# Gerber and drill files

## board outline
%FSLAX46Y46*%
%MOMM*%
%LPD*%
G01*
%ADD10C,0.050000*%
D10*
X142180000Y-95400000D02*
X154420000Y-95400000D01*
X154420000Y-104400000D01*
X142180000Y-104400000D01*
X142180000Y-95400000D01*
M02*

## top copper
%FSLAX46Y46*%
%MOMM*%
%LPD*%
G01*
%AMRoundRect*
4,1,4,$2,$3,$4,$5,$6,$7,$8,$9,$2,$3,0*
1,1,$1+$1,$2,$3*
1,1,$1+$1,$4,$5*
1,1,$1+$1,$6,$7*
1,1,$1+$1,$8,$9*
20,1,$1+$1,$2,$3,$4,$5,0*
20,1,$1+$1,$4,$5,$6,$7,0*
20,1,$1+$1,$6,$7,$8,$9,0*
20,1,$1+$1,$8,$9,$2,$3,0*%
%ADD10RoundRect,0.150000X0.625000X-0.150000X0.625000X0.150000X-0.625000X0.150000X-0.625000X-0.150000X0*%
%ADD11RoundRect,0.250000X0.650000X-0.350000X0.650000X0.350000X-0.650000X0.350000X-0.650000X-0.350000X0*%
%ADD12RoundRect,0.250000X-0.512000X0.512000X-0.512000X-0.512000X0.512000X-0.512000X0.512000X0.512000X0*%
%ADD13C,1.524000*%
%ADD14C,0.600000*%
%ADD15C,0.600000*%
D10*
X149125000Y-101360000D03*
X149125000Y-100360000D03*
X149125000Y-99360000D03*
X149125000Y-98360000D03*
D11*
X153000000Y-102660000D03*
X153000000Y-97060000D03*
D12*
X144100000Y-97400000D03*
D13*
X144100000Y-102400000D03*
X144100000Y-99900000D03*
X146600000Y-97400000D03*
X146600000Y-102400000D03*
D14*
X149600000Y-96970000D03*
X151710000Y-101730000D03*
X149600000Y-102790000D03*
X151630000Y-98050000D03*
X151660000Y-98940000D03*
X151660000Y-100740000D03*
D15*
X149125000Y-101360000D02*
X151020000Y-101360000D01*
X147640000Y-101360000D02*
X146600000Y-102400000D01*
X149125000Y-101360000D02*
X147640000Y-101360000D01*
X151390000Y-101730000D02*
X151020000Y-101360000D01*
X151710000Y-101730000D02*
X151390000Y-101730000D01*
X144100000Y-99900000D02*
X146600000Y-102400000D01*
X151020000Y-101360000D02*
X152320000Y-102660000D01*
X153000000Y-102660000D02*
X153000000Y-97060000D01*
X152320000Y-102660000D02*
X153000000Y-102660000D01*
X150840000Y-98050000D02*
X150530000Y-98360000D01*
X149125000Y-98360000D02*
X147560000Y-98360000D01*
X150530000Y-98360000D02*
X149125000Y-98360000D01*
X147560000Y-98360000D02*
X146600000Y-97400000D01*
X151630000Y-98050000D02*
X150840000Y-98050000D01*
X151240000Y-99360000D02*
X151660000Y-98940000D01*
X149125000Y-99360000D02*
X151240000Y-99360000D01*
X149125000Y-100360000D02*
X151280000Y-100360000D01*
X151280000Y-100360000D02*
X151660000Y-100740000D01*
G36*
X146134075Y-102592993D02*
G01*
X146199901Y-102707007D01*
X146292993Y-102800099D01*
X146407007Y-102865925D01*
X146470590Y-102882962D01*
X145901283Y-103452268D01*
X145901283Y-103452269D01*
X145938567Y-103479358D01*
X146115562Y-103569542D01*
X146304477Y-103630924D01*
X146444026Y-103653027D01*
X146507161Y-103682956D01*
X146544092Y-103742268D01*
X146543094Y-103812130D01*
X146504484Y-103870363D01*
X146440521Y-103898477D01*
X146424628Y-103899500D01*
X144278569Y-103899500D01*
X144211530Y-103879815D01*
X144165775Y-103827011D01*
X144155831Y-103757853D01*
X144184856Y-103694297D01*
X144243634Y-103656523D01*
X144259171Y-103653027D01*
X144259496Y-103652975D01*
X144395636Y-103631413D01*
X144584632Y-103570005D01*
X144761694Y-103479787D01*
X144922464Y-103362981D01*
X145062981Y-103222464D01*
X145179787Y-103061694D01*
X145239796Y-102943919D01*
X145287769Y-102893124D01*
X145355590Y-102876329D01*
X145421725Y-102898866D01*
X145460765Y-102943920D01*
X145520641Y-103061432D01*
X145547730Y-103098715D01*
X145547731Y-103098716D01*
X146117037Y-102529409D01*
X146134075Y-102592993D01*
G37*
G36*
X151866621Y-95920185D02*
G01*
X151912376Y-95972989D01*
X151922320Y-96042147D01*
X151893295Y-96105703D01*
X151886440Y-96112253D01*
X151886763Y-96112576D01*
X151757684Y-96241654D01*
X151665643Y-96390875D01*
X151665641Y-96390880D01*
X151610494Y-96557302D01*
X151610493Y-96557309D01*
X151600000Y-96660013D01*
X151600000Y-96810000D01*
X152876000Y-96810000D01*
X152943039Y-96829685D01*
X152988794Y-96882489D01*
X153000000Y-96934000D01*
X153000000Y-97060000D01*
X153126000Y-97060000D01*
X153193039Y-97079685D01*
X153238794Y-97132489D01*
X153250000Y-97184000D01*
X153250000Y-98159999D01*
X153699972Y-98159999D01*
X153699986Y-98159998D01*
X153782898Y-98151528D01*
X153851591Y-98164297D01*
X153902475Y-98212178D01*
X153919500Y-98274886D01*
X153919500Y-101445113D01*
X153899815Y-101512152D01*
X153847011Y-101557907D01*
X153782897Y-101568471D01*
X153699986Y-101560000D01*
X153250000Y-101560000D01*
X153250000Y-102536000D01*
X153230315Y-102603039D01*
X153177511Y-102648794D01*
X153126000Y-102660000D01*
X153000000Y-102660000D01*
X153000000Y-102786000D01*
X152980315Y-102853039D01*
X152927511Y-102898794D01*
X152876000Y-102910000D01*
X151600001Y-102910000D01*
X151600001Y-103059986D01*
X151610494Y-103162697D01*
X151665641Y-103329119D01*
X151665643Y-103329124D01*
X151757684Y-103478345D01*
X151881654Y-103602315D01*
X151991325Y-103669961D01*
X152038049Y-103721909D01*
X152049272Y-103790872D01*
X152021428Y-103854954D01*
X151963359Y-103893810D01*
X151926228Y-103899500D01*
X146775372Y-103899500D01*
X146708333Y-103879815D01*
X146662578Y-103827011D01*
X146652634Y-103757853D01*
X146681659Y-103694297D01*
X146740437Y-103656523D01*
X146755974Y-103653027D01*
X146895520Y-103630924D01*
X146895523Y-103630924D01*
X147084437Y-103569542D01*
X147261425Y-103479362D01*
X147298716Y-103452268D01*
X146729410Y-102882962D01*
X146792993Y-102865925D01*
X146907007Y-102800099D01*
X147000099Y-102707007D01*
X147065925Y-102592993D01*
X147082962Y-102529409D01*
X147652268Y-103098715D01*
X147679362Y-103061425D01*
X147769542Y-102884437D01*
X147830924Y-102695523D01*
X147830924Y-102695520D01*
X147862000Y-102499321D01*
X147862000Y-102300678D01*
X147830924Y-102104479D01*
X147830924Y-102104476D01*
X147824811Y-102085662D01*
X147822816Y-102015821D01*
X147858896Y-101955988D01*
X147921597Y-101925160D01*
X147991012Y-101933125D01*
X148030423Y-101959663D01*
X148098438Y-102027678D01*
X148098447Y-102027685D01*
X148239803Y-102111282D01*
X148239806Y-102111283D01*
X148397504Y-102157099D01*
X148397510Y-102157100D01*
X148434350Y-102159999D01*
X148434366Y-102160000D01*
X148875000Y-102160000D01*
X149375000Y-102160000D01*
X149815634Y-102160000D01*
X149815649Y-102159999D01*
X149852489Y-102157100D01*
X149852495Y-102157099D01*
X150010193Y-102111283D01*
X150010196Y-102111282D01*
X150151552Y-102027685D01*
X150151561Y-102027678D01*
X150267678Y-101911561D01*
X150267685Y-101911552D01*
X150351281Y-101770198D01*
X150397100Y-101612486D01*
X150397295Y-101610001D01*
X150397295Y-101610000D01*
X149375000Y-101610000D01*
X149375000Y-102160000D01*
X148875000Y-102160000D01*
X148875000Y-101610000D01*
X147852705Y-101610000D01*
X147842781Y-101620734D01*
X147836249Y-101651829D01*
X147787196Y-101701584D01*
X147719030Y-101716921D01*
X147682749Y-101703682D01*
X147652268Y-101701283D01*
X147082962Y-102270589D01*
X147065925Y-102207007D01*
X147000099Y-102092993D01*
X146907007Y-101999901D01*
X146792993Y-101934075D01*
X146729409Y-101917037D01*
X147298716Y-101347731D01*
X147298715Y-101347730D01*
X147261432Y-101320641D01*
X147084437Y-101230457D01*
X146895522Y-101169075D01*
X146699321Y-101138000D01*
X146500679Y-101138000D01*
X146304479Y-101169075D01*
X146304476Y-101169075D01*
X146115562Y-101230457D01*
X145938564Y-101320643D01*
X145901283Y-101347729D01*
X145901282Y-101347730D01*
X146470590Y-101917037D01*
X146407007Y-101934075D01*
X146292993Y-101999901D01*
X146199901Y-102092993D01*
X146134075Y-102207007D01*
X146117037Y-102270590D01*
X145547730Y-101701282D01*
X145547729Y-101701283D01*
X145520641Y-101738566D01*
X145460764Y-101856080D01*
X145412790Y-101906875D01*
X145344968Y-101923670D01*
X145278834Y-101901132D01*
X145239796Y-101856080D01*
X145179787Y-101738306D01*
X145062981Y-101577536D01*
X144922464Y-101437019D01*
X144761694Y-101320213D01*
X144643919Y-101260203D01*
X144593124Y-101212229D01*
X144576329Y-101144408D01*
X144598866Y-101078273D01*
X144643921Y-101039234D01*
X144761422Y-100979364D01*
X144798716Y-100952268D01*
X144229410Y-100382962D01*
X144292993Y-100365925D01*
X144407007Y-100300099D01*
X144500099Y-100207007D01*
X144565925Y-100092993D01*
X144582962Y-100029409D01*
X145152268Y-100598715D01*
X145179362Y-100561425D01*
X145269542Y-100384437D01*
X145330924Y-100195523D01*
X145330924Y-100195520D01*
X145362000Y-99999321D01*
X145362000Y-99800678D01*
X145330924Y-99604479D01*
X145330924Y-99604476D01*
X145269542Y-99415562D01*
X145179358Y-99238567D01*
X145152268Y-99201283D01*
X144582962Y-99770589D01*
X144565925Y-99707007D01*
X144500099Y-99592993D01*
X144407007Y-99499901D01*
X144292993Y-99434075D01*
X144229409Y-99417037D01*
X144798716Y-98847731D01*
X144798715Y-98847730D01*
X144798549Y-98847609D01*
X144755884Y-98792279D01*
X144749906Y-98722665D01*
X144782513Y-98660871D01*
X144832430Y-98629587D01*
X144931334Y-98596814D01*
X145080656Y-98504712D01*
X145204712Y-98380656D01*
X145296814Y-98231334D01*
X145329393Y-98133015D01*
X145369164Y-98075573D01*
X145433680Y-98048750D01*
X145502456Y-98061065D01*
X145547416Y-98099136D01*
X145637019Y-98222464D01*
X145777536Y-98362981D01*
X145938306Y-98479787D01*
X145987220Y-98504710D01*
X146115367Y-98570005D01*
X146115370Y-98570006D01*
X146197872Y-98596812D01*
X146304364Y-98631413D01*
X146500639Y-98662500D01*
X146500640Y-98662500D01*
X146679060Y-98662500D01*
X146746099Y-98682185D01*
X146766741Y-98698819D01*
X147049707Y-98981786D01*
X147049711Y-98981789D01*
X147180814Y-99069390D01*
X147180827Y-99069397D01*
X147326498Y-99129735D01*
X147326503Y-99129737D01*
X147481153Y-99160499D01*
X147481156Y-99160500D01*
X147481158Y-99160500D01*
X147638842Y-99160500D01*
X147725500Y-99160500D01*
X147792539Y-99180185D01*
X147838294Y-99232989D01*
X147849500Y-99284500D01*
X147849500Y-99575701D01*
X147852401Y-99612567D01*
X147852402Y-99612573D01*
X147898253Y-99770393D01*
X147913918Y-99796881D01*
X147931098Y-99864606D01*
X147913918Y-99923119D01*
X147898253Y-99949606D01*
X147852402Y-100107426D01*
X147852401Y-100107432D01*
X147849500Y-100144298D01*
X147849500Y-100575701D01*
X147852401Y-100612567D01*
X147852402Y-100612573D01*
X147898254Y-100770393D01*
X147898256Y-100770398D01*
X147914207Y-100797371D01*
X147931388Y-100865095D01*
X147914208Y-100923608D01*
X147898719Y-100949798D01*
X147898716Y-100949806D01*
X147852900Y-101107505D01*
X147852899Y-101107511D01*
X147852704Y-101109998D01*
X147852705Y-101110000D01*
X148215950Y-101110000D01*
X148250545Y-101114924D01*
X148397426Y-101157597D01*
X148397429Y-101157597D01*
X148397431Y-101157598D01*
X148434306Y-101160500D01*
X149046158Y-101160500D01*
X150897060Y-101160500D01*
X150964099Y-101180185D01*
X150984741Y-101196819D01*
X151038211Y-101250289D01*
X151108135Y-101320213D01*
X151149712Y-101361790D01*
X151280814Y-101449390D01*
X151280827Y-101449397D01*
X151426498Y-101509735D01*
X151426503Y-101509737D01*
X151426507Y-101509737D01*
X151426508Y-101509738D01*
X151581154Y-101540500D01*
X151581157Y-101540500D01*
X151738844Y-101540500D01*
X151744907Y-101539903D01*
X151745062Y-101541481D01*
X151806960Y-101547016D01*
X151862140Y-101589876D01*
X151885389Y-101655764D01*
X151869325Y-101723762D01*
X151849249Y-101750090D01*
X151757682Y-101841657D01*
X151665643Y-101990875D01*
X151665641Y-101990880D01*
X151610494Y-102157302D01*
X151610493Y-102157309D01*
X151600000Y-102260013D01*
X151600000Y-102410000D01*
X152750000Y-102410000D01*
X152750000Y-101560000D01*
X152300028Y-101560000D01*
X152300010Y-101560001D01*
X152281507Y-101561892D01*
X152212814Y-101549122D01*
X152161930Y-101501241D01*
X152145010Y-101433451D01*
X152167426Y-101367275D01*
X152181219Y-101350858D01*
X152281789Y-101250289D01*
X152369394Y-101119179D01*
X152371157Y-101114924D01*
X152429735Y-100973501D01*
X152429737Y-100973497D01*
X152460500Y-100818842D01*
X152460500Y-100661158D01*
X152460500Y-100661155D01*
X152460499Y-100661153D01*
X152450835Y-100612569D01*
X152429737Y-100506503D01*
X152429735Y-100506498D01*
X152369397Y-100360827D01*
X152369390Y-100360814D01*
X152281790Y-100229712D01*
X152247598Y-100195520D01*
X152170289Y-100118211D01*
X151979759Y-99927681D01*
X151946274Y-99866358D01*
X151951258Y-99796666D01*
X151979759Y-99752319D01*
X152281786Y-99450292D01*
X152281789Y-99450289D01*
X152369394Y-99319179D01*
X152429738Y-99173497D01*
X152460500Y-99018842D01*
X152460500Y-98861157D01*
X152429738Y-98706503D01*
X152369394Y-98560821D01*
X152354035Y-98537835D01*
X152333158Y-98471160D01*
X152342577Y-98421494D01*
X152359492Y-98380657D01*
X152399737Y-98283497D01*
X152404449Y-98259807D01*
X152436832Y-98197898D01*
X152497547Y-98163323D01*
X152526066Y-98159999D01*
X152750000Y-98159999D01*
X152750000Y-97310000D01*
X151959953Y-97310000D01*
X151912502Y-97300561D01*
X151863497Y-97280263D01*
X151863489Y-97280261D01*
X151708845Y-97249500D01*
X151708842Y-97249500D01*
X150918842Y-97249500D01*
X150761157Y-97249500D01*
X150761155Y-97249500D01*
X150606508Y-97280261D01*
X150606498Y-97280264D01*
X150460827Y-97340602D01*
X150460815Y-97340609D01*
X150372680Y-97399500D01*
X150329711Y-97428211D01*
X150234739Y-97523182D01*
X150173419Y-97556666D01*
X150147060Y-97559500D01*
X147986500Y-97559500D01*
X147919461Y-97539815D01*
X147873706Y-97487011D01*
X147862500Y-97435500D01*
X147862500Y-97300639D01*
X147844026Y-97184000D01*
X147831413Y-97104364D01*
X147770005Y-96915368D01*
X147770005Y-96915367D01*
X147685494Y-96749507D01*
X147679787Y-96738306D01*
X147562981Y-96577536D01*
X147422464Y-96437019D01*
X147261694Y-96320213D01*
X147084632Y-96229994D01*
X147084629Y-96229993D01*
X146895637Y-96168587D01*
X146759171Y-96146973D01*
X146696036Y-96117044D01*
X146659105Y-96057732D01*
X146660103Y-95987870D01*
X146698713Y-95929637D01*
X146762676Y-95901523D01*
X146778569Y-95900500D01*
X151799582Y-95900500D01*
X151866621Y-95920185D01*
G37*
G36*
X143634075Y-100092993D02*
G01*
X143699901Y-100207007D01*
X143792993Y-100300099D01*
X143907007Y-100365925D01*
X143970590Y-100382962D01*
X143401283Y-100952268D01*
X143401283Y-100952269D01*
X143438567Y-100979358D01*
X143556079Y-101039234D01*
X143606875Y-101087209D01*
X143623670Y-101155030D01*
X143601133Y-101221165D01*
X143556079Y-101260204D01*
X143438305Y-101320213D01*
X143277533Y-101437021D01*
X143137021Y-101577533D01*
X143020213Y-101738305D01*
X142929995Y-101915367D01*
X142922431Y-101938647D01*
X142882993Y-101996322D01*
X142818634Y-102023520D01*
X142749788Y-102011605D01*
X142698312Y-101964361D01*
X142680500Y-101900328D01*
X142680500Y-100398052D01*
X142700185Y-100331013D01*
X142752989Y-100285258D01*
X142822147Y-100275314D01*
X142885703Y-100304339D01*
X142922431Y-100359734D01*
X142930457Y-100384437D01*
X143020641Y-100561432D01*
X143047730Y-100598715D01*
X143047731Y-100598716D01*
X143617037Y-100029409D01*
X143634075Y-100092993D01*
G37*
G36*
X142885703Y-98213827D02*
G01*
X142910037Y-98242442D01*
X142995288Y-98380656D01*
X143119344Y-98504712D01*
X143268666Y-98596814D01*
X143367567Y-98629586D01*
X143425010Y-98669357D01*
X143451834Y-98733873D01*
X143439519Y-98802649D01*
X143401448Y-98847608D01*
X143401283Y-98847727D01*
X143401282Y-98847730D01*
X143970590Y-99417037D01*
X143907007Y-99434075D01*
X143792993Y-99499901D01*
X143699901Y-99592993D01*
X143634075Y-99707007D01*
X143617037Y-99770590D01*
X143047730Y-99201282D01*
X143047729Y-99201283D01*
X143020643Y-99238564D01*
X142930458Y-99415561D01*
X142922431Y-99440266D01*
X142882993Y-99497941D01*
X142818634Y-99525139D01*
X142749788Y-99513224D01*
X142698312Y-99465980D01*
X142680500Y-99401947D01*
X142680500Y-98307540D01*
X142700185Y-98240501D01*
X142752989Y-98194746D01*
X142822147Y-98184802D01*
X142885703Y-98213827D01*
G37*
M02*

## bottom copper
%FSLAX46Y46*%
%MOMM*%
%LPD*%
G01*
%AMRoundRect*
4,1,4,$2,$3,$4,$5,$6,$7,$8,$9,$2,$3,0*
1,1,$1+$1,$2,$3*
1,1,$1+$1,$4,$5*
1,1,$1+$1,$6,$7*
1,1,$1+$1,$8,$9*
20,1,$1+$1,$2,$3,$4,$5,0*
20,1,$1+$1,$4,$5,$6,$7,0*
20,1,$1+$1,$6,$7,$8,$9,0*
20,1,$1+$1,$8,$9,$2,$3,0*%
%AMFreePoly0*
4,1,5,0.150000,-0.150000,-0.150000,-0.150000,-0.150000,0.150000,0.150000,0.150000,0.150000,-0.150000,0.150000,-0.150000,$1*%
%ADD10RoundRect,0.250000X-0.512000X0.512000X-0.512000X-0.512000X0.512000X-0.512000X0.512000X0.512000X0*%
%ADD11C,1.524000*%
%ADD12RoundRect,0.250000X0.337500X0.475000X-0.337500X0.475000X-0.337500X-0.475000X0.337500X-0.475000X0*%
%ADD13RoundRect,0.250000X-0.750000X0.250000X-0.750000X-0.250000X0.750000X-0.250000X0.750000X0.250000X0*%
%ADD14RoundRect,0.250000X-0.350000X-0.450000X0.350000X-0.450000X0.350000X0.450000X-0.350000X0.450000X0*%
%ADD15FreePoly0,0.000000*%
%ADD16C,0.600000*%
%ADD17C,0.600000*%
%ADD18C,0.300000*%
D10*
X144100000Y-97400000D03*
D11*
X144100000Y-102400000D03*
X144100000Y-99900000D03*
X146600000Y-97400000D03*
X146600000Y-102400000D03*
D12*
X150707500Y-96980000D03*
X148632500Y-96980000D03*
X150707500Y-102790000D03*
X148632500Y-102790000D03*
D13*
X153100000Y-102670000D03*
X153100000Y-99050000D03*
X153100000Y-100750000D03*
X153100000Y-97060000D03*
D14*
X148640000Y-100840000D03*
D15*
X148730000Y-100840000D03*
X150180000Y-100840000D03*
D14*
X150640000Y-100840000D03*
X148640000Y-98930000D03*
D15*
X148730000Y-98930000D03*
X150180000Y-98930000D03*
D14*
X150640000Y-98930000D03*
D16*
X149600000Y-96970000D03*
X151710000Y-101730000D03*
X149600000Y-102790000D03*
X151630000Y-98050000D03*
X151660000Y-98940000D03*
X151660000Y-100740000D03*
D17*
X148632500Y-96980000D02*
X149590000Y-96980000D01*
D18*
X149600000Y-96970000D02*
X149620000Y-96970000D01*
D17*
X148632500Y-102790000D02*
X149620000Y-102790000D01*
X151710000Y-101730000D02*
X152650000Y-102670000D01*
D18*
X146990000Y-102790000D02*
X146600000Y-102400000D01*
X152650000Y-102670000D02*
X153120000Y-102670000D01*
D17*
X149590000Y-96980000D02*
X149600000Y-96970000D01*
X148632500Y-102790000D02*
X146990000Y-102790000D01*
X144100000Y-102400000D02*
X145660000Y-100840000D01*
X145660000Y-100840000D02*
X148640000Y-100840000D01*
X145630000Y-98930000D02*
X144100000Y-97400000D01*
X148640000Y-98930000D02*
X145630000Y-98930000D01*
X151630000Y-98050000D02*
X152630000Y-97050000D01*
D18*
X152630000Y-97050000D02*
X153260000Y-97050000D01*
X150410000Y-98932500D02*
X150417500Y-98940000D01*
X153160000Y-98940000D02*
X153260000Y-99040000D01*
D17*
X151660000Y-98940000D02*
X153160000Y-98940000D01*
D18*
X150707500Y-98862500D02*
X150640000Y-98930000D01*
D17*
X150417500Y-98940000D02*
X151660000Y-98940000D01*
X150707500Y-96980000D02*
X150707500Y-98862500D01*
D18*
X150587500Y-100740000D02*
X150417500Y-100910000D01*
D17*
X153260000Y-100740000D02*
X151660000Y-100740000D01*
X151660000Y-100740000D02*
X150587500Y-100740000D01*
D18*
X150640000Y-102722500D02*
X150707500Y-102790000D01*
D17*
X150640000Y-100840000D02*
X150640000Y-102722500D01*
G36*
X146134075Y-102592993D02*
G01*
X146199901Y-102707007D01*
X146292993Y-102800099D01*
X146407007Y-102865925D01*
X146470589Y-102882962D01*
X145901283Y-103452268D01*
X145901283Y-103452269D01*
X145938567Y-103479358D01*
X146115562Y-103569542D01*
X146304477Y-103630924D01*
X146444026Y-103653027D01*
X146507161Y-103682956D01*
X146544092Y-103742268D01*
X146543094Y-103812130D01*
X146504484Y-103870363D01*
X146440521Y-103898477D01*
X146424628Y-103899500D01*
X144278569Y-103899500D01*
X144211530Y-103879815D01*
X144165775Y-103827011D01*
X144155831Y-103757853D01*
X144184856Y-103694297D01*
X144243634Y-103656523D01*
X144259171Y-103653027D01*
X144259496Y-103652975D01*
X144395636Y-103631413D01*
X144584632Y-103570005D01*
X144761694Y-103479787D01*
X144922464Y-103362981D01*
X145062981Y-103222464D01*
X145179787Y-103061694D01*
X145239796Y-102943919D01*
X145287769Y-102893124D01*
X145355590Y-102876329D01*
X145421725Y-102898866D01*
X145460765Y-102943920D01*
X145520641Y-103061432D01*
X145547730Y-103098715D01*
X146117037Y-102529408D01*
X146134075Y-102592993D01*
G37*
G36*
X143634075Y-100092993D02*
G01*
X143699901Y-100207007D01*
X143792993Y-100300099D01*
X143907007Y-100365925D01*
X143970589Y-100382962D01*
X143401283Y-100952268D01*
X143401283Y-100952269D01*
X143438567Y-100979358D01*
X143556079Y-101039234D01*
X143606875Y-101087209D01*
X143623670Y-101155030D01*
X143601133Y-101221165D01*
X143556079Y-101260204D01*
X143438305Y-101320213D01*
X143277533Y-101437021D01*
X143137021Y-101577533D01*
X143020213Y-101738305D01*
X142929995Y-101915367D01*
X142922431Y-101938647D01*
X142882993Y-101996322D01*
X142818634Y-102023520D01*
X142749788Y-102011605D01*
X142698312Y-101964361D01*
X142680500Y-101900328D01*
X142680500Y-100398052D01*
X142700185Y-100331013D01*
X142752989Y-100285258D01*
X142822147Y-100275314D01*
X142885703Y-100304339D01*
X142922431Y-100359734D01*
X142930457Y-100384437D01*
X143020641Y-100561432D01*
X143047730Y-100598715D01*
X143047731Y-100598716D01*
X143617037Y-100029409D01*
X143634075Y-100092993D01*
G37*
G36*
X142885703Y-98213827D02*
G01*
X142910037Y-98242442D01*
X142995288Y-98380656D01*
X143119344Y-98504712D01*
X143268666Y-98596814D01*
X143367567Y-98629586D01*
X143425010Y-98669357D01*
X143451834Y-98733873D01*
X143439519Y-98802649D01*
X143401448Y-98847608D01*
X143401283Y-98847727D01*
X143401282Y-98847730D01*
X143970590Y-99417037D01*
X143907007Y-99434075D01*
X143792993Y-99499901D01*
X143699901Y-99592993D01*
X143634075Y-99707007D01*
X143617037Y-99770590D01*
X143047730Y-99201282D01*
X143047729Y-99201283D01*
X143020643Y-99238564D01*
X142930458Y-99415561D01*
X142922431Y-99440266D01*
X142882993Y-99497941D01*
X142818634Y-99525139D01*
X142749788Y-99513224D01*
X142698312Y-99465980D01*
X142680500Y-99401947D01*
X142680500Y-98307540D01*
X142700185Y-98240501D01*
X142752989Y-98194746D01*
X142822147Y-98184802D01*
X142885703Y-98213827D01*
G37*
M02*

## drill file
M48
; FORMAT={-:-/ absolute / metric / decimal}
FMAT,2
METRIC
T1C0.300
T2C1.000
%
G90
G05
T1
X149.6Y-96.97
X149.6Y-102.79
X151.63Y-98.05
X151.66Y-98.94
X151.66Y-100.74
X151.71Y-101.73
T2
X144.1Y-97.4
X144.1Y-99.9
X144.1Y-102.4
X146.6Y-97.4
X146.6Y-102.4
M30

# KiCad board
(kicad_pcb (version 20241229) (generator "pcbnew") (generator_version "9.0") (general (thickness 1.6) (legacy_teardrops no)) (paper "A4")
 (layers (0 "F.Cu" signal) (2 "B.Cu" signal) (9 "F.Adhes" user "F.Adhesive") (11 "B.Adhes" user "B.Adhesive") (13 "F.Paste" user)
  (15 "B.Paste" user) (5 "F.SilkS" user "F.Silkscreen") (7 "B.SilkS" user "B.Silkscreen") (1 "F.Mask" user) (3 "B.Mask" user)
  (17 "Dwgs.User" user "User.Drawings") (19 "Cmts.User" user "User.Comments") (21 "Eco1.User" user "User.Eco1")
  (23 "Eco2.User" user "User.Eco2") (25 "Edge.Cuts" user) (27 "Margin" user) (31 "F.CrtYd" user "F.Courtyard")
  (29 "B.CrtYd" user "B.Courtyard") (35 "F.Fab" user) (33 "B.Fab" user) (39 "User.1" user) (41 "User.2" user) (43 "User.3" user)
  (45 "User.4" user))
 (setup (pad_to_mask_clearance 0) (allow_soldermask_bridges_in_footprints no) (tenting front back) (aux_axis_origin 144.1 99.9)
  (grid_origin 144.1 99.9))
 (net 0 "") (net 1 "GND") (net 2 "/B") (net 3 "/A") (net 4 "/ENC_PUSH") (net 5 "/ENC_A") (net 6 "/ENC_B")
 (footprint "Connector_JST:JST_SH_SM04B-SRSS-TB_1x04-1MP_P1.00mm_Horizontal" (layer "F.Cu") (at 151.125 99.86 90)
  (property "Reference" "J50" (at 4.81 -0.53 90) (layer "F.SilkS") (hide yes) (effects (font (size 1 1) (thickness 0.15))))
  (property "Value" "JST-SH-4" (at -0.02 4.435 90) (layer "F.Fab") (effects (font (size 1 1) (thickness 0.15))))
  (pad "1" smd roundrect (at -1.5 -2 90) (size 0.6 1.55) (layers "F.Cu" "F.Mask" "F.Paste") (roundrect_rratio 0.25) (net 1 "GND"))
  (pad "2" smd roundrect (at -0.5 -2 90) (size 0.6 1.55) (layers "F.Cu" "F.Mask" "F.Paste") (roundrect_rratio 0.25) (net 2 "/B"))
  (pad "3" smd roundrect (at 0.5 -2 90) (size 0.6 1.55) (layers "F.Cu" "F.Mask" "F.Paste") (roundrect_rratio 0.25) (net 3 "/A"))
  (pad "4" smd roundrect (at 1.5 -2 90) (size 0.6 1.55) (layers "F.Cu" "F.Mask" "F.Paste") (roundrect_rratio 0.25) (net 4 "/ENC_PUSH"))
  (pad "MP" smd roundrect (at -2.8 1.875 90) (size 1.2 1.8) (layers "F.Cu" "F.Mask" "F.Paste") (roundrect_rratio 0.208333) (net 1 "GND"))
  (pad "MP" smd roundrect (at 2.8 1.875 90) (size 1.2 1.8) (layers "F.Cu" "F.Mask" "F.Paste") (roundrect_rratio 0.208333) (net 1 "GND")))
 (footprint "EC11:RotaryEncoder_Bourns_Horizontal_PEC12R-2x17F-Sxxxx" (layer "F.Cu") (at 144.1 97.4)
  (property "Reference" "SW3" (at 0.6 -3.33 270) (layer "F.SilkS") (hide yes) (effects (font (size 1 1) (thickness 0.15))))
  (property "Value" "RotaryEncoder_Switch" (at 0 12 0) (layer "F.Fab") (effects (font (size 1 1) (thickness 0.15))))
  (pad "A" thru_hole roundrect (at 0 0 270) (size 1.524 1.524) (drill 1) (layers "*.Cu" "*.Mask") (remove_unused_layers no)
   (roundrect_rratio 0.1640419948) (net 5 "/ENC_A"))
  (pad "B" thru_hole circle (at 0 5 270) (size 1.524 1.524) (drill 1) (layers "*.Cu" "*.Mask") (remove_unused_layers no) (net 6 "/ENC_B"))
  (pad "C" thru_hole circle (at 0 2.5 270) (size 1.524 1.524) (drill 1) (layers "*.Cu" "*.Mask") (remove_unused_layers no) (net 1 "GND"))
  (pad "S1" thru_hole circle (at 2.5 0 270) (size 1.524 1.524) (drill 1) (layers "*.Cu" "*.Mask") (remove_unused_layers no)
   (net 4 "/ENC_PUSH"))
  (pad "S2" thru_hole circle (at 2.5 5 270) (size 1.524 1.524) (drill 1) (layers "*.Cu" "*.Mask") (remove_unused_layers no) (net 1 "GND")))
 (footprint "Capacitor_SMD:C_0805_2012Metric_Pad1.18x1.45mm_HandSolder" (layer "B.Cu") (at 149.67 96.98 180)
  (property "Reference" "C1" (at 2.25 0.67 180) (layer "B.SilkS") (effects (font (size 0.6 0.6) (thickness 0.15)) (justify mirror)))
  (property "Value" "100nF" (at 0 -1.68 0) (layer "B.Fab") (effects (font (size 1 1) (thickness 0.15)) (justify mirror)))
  (pad "1" smd roundrect (at -1.0375 0 180) (size 1.175 1.45) (layers "B.Cu" "B.Mask" "B.Paste") (roundrect_rratio 0.212766) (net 3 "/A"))
  (pad "2" smd roundrect (at 1.0375 0 180) (size 1.175 1.45) (layers "B.Cu" "B.Mask" "B.Paste") (roundrect_rratio 0.212766) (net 1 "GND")))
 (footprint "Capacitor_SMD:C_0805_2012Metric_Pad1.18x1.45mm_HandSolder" (layer "B.Cu") (at 149.67 102.79 180)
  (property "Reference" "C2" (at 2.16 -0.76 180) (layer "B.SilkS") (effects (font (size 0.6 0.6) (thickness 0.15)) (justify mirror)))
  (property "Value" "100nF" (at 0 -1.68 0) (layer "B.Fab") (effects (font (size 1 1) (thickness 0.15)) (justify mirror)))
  (pad "1" smd roundrect (at -1.0375 0 180) (size 1.175 1.45) (layers "B.Cu" "B.Mask" "B.Paste") (roundrect_rratio 0.212766) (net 2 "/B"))
  (pad "2" smd roundrect (at 1.0375 0 180) (size 1.175 1.45) (layers "B.Cu" "B.Mask" "B.Paste") (roundrect_rratio 0.212766) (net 1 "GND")))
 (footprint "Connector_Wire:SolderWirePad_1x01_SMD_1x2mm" (layer "B.Cu") (at 153.1 102.67 -90)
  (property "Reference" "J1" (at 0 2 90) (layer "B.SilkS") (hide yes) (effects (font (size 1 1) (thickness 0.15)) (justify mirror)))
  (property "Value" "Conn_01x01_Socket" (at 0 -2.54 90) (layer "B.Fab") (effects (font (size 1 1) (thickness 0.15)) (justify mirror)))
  (pad "1" smd roundrect (at 0 0 270) (size 1 2) (layers "B.Cu" "B.Mask") (roundrect_rratio 0.25) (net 1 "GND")))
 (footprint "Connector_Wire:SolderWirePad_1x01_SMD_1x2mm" (layer "B.Cu") (at 153.1 99.05 -90)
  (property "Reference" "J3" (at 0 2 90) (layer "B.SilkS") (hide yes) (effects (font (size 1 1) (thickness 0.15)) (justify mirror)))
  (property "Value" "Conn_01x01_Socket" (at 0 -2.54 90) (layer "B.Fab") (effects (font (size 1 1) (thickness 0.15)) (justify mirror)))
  (pad "1" smd roundrect (at 0 0 270) (size 1 2) (layers "B.Cu" "B.Mask") (roundrect_rratio 0.25) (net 3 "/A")))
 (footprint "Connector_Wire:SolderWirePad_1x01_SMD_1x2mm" (layer "B.Cu") (at 153.1 100.75 -90)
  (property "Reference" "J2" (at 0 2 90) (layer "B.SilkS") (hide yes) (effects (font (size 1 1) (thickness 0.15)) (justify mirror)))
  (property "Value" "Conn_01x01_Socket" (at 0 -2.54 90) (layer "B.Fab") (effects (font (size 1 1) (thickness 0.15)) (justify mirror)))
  (pad "1" smd roundrect (at 0 0 270) (size 1 2) (layers "B.Cu" "B.Mask") (roundrect_rratio 0.25) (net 2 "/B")))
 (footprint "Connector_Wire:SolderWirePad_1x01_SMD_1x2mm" (layer "B.Cu") (at 153.1 97.06 -90)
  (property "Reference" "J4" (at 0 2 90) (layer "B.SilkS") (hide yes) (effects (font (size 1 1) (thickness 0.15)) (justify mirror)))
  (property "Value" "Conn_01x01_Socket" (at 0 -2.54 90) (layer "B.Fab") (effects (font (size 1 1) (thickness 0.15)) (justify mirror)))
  (pad "1" smd roundrect (at 0 0 270) (size 1 2) (layers "B.Cu" "B.Mask") (roundrect_rratio 0.25) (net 4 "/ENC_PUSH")))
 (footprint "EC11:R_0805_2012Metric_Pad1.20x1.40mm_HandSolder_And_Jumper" (layer "B.Cu") (at 149.64 100.84)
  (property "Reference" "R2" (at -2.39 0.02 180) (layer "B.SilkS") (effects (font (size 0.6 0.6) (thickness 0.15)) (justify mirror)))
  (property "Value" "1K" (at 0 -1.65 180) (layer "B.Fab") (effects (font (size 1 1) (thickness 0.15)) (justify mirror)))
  (pad "1" smd roundrect (at -1 0) (size 1.2 1.4) (layers "B.Cu" "B.Mask" "B.Paste") (roundrect_rratio 0.208333) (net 6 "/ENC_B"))
  (pad "1" smd custom (at -0.91 0) (size 0.3 0.3) (layers "B.Cu" "B.Mask") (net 6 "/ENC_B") (zone_connect 2) (thermal_bridge_angle 45)
   (options (clearance outline) (anchor rect)) (primitives))
  (pad "2" smd custom (at 0.54 0) (size 0.3 0.3) (layers "B.Cu" "B.Mask") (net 2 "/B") (zone_connect 2) (thermal_bridge_angle 45)
   (options (clearance outline) (anchor rect)) (primitives))
  (pad "2" smd roundrect (at 1 0) (size 1.2 1.4) (layers "B.Cu" "B.Mask" "B.Paste") (roundrect_rratio 0.208333) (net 2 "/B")))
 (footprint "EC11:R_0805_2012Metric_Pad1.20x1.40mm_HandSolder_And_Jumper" (layer "B.Cu") (at 149.64 98.93)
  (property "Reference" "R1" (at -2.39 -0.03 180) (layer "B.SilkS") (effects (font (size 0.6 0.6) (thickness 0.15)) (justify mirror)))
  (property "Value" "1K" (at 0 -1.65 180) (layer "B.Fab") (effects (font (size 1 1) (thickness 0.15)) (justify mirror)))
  (pad "1" smd roundrect (at -1 0) (size 1.2 1.4) (layers "B.Cu" "B.Mask" "B.Paste") (roundrect_rratio 0.208333) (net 5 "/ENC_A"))
  (pad "1" smd custom (at -0.91 0) (size 0.3 0.3) (layers "B.Cu" "B.Mask") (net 5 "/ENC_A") (zone_connect 2) (thermal_bridge_angle 45)
   (options (clearance outline) (anchor rect)) (primitives))
  (pad "2" smd custom (at 0.54 0) (size 0.3 0.3) (layers "B.Cu" "B.Mask") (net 3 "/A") (zone_connect 2) (thermal_bridge_angle 45)
   (options (clearance outline) (anchor rect)) (primitives))
  (pad "2" smd roundrect (at 1 0) (size 1.2 1.4) (layers "B.Cu" "B.Mask" "B.Paste") (roundrect_rratio 0.208333) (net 3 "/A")))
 (gr_rect (start 142.18 95.4) (end 154.42 104.4) (stroke (width 0.05) (type solid)) (fill no) (layer "Edge.Cuts"))
 (segment (start 149.125 101.36) (end 151.02 101.36) (width 0.6) (layer "F.Cu") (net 1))
 (segment (start 147.64 101.36) (end 146.6 102.4) (width 0.6) (layer "F.Cu") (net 1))
 (segment (start 149.125 101.36) (end 147.64 101.36) (width 0.6) (layer "F.Cu") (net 1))
 (segment (start 151.39 101.73) (end 151.02 101.36) (width 0.6) (layer "F.Cu") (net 1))
 (segment (start 151.71 101.73) (end 151.39 101.73) (width 0.6) (layer "F.Cu") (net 1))
 (segment (start 144.1 99.9) (end 146.6 102.4) (width 0.6) (layer "F.Cu") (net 1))
 (segment (start 151.02 101.36) (end 152.32 102.66) (width 0.6) (layer "F.Cu") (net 1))
 (segment (start 153 102.66) (end 153 97.06) (width 0.6) (layer "F.Cu") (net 1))
 (segment (start 152.32 102.66) (end 153 102.66) (width 0.6) (layer "F.Cu") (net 1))
 (via (at 149.6 96.97) (size 0.6) (drill 0.3) (layers "F.Cu" "B.Cu") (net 1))
 (via (at 151.71 101.73) (size 0.6) (drill 0.3) (layers "F.Cu" "B.Cu") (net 1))
 (via (at 149.6 102.79) (size 0.6) (drill 0.3) (layers "F.Cu" "B.Cu") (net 1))
 (segment (start 148.6325 96.98) (end 149.59 96.98) (width 0.6) (layer "B.Cu") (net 1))
 (segment (start 149.6 96.97) (end 149.62 96.97) (width 0.3) (layer "B.Cu") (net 1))
 (segment (start 148.6325 102.79) (end 149.62 102.79) (width 0.6) (layer "B.Cu") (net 1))
 (segment (start 151.71 101.73) (end 152.65 102.67) (width 0.6) (layer "B.Cu") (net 1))
 (segment (start 146.99 102.79) (end 146.6 102.4) (width 0.3) (layer "B.Cu") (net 1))
 (segment (start 152.65 102.67) (end 153.12 102.67) (width 0.3) (layer "B.Cu") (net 1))
 (segment (start 149.59 96.98) (end 149.6 96.97) (width 0.6) (layer "B.Cu") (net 1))
 (segment (start 148.6325 102.79) (end 146.99 102.79) (width 0.6) (layer "B.Cu") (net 1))
 (segment (start 144.1 102.4) (end 145.66 100.84) (width 0.6) (layer "B.Cu") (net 6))
 (segment (start 145.66 100.84) (end 148.64 100.84) (width 0.6) (layer "B.Cu") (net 6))
 (segment (start 145.63 98.93) (end 144.1 97.4) (width 0.6) (layer "B.Cu") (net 5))
 (segment (start 148.64 98.93) (end 145.63 98.93) (width 0.6) (layer "B.Cu") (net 5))
 (segment (start 150.84 98.05) (end 150.53 98.36) (width 0.6) (layer "F.Cu") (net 4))
 (segment (start 149.125 98.36) (end 147.56 98.36) (width 0.6) (layer "F.Cu") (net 4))
 (segment (start 150.53 98.36) (end 149.125 98.36) (width 0.6) (layer "F.Cu") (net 4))
 (segment (start 147.56 98.36) (end 146.6 97.4) (width 0.6) (layer "F.Cu") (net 4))
 (segment (start 151.63 98.05) (end 150.84 98.05) (width 0.6) (layer "F.Cu") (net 4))
 (via (at 151.63 98.05) (size 0.6) (drill 0.3) (layers "F.Cu" "B.Cu") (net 4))
 (segment (start 151.63 98.05) (end 152.63 97.05) (width 0.6) (layer "B.Cu") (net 4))
 (segment (start 152.63 97.05) (end 153.26 97.05) (width 0.3) (layer "B.Cu") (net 4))
 (segment (start 151.24 99.36) (end 151.66 98.94) (width 0.6) (layer "F.Cu") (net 3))
 (segment (start 149.125 99.36) (end 151.24 99.36) (width 0.6) (layer "F.Cu") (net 3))
 (via (at 151.66 98.94) (size 0.6) (drill 0.3) (layers "F.Cu" "B.Cu") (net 3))
 (segment (start 150.41 98.9325) (end 150.4175 98.94) (width 0.3) (layer "B.Cu") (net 3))
 (segment (start 153.16 98.94) (end 153.26 99.04) (width 0.3) (layer "B.Cu") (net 3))
 (segment (start 151.66 98.94) (end 153.16 98.94) (width 0.6) (layer "B.Cu") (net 3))
 (segment (start 150.7075 98.8625) (end 150.64 98.93) (width 0.3) (layer "B.Cu") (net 3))
 (segment (start 150.4175 98.94) (end 151.66 98.94) (width 0.6) (layer "B.Cu") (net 3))
 (segment (start 150.7075 96.98) (end 150.7075 98.8625) (width 0.6) (layer "B.Cu") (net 3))
 (segment (start 149.125 100.36) (end 151.28 100.36) (width 0.6) (layer "F.Cu") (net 2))
 (segment (start 151.28 100.36) (end 151.66 100.74) (width 0.6) (layer "F.Cu") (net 2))
 (via (at 151.66 100.74) (size 0.6) (drill 0.3) (layers "F.Cu" "B.Cu") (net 2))
 (segment (start 150.5875 100.74) (end 150.4175 100.91) (width 0.3) (layer "B.Cu") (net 2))
 (segment (start 153.26 100.74) (end 151.66 100.74) (width 0.6) (layer "B.Cu") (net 2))
 (segment (start 151.66 100.74) (end 150.5875 100.74) (width 0.6) (layer "B.Cu") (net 2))
 (segment (start 150.64 102.7225) (end 150.7075 102.79) (width 0.3) (layer "B.Cu") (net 2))
 (segment (start 150.64 100.84) (end 150.64 102.7225) (width 0.6) (layer "B.Cu") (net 2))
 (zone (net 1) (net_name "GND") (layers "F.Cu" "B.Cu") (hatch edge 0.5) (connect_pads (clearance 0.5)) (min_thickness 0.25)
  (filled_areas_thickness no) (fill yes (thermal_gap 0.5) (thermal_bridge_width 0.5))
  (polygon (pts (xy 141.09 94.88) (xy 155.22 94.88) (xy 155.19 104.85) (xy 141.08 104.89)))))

